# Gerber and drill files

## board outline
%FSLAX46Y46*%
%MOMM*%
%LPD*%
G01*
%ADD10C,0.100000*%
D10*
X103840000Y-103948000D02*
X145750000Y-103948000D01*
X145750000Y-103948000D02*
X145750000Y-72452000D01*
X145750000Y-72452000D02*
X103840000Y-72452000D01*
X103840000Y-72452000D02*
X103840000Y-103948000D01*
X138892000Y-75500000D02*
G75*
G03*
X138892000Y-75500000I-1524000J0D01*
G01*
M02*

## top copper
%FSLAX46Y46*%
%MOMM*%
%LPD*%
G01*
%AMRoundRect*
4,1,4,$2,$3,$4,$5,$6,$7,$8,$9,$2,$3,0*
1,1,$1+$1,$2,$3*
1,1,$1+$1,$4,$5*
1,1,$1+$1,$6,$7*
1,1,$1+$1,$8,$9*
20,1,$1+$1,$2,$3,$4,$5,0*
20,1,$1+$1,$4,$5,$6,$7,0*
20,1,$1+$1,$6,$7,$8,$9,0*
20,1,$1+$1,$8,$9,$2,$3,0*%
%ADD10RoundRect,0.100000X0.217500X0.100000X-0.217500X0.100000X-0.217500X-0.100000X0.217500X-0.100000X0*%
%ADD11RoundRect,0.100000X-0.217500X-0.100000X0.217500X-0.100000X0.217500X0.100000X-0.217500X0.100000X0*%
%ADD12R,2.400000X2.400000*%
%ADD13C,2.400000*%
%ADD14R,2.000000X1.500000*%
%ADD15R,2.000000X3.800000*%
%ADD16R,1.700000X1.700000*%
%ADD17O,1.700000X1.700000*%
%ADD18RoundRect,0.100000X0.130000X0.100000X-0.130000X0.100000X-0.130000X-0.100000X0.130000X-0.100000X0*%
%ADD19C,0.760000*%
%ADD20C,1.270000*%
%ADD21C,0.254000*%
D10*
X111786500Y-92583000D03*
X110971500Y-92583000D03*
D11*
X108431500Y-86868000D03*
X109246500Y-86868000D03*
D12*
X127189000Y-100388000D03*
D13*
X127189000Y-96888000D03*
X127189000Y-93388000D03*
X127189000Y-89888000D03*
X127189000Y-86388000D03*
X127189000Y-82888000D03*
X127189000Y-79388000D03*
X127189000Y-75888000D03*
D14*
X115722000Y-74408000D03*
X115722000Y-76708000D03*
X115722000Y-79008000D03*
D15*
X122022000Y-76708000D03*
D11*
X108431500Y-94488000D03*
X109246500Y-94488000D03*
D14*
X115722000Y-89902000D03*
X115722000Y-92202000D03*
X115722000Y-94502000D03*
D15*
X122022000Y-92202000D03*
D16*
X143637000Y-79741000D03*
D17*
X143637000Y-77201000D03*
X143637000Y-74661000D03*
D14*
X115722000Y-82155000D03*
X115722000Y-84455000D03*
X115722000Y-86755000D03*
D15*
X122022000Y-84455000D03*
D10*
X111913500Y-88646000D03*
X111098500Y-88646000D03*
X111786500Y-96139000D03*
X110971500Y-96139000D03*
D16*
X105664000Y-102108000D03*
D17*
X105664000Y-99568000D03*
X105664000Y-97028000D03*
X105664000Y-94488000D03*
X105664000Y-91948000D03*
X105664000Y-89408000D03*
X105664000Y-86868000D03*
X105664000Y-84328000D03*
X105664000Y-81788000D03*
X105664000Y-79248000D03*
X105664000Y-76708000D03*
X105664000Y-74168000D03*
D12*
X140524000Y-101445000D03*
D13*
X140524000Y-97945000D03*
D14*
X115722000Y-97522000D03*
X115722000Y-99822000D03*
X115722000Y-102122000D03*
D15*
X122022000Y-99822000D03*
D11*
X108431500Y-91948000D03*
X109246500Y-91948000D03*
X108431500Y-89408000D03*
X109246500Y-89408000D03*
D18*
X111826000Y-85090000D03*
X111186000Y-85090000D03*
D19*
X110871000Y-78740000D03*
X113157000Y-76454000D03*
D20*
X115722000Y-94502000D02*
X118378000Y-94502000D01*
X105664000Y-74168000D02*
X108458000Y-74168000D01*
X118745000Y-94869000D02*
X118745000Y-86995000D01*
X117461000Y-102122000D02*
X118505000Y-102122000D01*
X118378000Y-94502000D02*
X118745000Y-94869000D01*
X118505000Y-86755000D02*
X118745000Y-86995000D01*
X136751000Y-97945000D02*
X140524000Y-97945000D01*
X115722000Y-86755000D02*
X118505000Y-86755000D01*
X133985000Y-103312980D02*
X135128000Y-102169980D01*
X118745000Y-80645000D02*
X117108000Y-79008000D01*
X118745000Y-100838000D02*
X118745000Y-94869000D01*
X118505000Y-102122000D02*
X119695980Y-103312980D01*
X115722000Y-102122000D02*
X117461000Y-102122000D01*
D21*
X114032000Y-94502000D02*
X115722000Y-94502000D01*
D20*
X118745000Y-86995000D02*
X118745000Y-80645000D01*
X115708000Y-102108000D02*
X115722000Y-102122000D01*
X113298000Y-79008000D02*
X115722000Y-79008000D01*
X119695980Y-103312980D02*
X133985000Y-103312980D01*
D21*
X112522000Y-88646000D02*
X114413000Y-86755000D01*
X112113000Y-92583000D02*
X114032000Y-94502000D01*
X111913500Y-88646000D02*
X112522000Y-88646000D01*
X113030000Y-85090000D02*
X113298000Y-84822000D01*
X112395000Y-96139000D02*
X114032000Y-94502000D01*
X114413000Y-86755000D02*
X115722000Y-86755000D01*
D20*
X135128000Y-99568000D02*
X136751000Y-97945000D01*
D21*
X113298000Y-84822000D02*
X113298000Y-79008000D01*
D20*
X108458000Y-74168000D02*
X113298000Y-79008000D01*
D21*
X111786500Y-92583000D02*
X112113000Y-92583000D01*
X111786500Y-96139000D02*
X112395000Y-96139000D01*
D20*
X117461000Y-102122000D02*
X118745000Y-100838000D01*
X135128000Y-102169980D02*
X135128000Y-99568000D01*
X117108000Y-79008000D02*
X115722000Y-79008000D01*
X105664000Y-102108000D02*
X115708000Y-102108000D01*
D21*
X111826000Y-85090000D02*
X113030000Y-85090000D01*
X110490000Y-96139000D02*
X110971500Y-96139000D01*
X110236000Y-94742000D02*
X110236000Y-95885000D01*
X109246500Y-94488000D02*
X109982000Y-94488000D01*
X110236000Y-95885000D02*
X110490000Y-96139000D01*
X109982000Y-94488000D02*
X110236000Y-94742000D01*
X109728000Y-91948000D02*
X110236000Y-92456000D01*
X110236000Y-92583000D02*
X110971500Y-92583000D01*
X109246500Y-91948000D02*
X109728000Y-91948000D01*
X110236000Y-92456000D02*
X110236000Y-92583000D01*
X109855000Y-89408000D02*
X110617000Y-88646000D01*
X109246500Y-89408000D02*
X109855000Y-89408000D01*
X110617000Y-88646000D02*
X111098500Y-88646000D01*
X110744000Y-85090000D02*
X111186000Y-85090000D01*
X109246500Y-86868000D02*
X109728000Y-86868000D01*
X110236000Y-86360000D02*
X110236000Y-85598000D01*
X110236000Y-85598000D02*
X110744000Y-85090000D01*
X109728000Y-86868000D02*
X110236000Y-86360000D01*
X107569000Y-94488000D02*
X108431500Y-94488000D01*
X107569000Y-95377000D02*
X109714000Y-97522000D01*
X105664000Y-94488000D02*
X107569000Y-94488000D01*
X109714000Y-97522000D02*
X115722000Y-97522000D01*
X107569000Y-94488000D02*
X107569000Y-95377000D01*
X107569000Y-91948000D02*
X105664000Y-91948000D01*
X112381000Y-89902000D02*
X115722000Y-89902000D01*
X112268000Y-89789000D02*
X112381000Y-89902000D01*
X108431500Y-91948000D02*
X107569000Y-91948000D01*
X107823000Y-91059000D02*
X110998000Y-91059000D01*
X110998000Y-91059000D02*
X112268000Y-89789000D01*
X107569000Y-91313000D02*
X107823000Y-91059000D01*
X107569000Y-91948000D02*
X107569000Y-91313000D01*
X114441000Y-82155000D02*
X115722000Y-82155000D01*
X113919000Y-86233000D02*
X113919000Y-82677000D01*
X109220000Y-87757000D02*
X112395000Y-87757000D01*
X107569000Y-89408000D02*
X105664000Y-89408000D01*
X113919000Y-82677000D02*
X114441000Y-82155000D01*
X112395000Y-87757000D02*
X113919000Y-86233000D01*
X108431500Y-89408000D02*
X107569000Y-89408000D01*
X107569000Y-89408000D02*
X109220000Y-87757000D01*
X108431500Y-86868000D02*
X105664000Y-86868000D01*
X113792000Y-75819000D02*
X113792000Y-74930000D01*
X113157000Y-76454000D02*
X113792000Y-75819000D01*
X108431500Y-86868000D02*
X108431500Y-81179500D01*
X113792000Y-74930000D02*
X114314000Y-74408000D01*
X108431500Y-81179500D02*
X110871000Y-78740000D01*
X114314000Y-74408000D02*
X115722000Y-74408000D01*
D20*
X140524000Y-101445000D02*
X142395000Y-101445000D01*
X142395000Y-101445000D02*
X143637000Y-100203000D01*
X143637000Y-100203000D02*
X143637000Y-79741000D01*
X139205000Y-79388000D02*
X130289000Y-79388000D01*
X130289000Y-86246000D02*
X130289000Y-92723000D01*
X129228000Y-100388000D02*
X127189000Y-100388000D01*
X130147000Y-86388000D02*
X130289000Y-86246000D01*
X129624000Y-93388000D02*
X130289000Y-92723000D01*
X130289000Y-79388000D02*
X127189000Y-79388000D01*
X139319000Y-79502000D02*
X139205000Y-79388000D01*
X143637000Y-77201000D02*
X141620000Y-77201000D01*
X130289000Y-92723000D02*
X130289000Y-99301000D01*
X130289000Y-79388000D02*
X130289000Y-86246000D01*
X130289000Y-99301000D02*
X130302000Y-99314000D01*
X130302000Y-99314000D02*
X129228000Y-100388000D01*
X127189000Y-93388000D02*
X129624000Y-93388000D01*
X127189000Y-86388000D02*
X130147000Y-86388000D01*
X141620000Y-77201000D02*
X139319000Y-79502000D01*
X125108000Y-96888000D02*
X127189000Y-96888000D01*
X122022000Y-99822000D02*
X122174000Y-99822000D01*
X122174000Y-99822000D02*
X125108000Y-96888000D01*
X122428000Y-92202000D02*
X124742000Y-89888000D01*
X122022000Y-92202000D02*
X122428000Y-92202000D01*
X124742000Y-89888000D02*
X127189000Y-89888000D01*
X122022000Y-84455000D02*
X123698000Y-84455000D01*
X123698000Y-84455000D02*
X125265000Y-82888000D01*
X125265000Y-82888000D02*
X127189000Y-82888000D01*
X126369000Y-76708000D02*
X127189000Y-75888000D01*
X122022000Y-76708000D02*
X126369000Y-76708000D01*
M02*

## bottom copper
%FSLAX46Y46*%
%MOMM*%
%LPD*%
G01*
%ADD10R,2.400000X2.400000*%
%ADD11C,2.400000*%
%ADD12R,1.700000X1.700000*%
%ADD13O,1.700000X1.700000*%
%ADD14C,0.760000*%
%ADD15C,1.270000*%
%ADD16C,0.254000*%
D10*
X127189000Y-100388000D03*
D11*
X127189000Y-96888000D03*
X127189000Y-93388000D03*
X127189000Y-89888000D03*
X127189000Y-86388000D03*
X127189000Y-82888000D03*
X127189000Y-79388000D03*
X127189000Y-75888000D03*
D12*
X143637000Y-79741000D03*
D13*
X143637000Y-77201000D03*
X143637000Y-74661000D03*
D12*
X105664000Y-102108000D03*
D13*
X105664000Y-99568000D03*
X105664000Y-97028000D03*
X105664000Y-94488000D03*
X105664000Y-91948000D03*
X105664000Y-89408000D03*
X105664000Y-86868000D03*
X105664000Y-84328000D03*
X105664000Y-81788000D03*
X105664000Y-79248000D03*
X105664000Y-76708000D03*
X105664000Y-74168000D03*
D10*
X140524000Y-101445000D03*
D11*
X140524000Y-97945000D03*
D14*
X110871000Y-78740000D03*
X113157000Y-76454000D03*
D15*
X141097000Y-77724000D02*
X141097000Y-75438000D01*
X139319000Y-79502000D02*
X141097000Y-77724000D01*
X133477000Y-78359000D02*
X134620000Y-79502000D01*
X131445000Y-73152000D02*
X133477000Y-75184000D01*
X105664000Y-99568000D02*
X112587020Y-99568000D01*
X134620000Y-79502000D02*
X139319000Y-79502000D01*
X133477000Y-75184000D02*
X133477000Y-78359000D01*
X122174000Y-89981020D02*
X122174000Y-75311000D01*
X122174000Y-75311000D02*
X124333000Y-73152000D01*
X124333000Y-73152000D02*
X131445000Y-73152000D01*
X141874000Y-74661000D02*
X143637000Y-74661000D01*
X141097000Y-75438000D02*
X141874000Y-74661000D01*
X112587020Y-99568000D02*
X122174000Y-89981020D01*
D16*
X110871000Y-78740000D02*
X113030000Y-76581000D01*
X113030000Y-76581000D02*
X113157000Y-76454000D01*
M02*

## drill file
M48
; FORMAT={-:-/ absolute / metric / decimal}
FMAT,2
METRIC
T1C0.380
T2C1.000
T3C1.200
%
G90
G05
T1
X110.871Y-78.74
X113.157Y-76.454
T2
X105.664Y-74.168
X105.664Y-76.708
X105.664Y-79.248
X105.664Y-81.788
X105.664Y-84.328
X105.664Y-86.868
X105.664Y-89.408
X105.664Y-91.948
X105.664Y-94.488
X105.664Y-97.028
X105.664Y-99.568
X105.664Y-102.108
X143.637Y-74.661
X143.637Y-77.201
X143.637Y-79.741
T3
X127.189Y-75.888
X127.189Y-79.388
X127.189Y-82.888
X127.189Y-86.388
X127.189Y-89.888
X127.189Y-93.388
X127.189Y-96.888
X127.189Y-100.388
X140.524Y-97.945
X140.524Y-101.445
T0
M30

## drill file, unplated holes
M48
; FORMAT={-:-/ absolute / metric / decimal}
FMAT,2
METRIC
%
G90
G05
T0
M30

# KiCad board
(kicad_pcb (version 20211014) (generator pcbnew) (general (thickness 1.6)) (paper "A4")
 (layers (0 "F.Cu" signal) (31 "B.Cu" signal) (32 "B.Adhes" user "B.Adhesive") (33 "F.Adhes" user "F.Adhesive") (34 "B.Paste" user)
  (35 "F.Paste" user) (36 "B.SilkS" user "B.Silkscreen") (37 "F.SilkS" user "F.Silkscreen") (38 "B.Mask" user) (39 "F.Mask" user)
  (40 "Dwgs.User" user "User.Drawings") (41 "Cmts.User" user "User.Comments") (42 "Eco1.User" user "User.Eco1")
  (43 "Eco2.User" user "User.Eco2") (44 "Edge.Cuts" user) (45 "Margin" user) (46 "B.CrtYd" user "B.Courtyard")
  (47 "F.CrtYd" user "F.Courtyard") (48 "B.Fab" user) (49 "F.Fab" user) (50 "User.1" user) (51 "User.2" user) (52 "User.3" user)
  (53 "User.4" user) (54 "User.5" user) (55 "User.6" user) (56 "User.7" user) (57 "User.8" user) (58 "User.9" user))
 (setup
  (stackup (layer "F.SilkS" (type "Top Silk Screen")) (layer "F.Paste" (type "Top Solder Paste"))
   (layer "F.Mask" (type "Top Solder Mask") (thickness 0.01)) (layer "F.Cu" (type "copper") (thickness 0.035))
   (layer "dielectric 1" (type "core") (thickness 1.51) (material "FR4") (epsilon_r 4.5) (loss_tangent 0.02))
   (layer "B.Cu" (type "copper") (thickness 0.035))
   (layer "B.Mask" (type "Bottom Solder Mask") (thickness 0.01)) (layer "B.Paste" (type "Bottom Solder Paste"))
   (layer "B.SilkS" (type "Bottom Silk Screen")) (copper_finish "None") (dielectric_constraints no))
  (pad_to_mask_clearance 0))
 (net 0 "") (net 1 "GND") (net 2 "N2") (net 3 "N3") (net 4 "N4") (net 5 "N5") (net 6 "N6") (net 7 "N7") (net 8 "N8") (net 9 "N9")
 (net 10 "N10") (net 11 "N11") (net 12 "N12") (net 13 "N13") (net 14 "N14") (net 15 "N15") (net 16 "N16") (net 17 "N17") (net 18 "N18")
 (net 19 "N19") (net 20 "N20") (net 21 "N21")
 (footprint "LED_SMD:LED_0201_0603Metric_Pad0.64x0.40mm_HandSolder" (layer "F.Cu") (at 111.379 92.583 180)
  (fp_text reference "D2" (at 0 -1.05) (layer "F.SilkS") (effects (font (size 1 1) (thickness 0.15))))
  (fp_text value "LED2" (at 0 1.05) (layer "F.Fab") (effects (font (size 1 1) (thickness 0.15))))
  (pad "" smd roundrect locked (at 0.4325 0 180) (size 0.458 0.36) (layers "F.Paste") (roundrect_rratio 0.25))
  (pad "" smd roundrect locked (at -0.4325 0 180) (size 0.458 0.36) (layers "F.Paste") (roundrect_rratio 0.25))
  (pad "1" smd roundrect locked (at -0.4075 0 180) (size 0.635 0.4) (layers "F.Cu" "F.Mask") (roundrect_rratio 0.25) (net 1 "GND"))
  (pad "2" smd roundrect locked (at 0.4075 0 180) (size 0.635 0.4) (layers "F.Cu" "F.Mask") (roundrect_rratio 0.25) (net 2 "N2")))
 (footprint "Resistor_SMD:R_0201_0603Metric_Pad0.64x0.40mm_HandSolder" (layer "F.Cu") (at 108.839 86.868)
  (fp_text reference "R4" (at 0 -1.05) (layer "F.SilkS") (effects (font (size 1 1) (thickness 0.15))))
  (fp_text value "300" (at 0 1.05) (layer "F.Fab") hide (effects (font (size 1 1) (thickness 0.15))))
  (pad "" smd roundrect locked (at 0.4325 0) (size 0.458 0.36) (layers "F.Paste") (roundrect_rratio 0.25))
  (pad "" smd roundrect locked (at -0.4325 0) (size 0.458 0.36) (layers "F.Paste") (roundrect_rratio 0.25))
  (pad "1" smd roundrect locked (at -0.4075 0) (size 0.635 0.4) (layers "F.Cu" "F.Mask") (roundrect_rratio 0.25) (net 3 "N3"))
  (pad "2" smd roundrect locked (at 0.4075 0) (size 0.635 0.4) (layers "F.Cu" "F.Mask") (roundrect_rratio 0.25) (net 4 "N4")))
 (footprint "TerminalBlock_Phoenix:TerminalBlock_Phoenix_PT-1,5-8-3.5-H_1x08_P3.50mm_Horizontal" (layer "F.Cu") (at 127.189 100.388 90)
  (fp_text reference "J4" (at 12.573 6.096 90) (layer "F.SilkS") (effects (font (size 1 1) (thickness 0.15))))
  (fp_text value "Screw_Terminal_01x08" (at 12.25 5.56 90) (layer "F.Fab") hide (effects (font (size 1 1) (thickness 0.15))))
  (pad "1" thru_hole rect locked (at 0 0 90) (size 2.4 2.4) (drill 1.2) (layers *.Cu *.Mask) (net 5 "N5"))
  (pad "2" thru_hole circle locked (at 3.5 0 90) (size 2.4 2.4) (drill 1.2) (layers *.Cu *.Mask) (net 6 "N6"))
  (pad "3" thru_hole circle locked (at 7 0 90) (size 2.4 2.4) (drill 1.2) (layers *.Cu *.Mask) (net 5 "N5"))
  (pad "4" thru_hole circle locked (at 10.5 0 90) (size 2.4 2.4) (drill 1.2) (layers *.Cu *.Mask) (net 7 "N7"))
  (pad "5" thru_hole circle locked (at 14 0 90) (size 2.4 2.4) (drill 1.2) (layers *.Cu *.Mask) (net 5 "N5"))
  (pad "6" thru_hole circle locked (at 17.5 0 90) (size 2.4 2.4) (drill 1.2) (layers *.Cu *.Mask) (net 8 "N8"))
  (pad "7" thru_hole circle locked (at 21 0 90) (size 2.4 2.4) (drill 1.2) (layers *.Cu *.Mask) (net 5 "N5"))
  (pad "8" thru_hole circle locked (at 24.5 0 90) (size 2.4 2.4) (drill 1.2) (layers *.Cu *.Mask) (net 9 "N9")))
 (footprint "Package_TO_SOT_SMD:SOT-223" (layer "F.Cu") (at 118.872 76.708)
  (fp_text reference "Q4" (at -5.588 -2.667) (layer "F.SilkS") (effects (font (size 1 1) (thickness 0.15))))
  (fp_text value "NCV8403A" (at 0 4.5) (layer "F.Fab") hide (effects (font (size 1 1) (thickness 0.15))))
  (pad "1" smd rect locked (at -3.15 -2.3) (size 2 1.5) (layers "F.Cu" "F.Paste" "F.Mask") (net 3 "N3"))
  (pad "2" smd rect locked (at -3.15 0) (size 2 1.5) (layers "F.Cu" "F.Paste" "F.Mask"))
  (pad "3" smd rect locked (at -3.15 2.3) (size 2 1.5) (layers "F.Cu" "F.Paste" "F.Mask") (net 1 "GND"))
  (pad "4" smd rect locked (at 3.15 0) (size 2 3.8) (layers "F.Cu" "F.Paste" "F.Mask") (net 9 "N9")))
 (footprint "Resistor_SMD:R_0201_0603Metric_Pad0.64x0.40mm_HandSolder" (layer "F.Cu") (at 108.839 94.488)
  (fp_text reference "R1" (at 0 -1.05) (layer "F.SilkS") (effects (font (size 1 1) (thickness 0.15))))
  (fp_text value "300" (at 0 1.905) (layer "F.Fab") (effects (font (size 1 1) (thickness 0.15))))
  (pad "" smd roundrect locked (at -0.4325 0) (size 0.458 0.36) (layers "F.Paste") (roundrect_rratio 0.25))
  (pad "" smd roundrect locked (at 0.4325 0) (size 0.458 0.36) (layers "F.Paste") (roundrect_rratio 0.25))
  (pad "1" smd roundrect locked (at -0.4075 0) (size 0.635 0.4) (layers "F.Cu" "F.Mask") (roundrect_rratio 0.25) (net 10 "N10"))
  (pad "2" smd roundrect locked (at 0.4075 0) (size 0.635 0.4) (layers "F.Cu" "F.Mask") (roundrect_rratio 0.25) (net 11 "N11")))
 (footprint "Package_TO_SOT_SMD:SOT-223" (layer "F.Cu") (at 118.872 92.202)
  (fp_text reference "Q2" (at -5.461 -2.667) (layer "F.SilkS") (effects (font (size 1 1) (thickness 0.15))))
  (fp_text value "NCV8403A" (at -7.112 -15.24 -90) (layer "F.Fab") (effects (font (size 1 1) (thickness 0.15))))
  (pad "1" smd rect locked (at -3.15 -2.3) (size 2 1.5) (layers "F.Cu" "F.Paste" "F.Mask") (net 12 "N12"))
  (pad "2" smd rect locked (at -3.15 0) (size 2 1.5) (layers "F.Cu" "F.Paste" "F.Mask"))
  (pad "3" smd rect locked (at -3.15 2.3) (size 2 1.5) (layers "F.Cu" "F.Paste" "F.Mask") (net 1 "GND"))
  (pad "4" smd rect locked (at 3.15 0) (size 2 3.8) (layers "F.Cu" "F.Paste" "F.Mask") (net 7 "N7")))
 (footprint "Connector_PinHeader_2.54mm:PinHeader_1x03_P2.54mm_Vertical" (layer "F.Cu") (at 143.637 79.741 180)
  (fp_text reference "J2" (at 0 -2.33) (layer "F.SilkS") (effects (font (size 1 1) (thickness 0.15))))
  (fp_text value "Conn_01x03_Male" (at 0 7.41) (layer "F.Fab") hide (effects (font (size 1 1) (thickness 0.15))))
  (pad "1" thru_hole rect locked (at 0 0 180) (size 1.7 1.7) (drill 1) (layers *.Cu *.Mask) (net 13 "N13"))
  (pad "2" thru_hole oval locked (at 0 2.54 180) (size 1.7 1.7) (drill 1) (layers *.Cu *.Mask) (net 5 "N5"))
  (pad "3" thru_hole oval locked (at 0 5.08 180) (size 1.7 1.7) (drill 1) (layers *.Cu *.Mask) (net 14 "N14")))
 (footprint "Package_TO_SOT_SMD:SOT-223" (layer "F.Cu") (at 118.872 84.455)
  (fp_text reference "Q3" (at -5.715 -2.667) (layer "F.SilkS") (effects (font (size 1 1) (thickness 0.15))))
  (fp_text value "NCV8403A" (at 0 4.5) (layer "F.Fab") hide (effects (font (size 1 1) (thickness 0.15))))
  (pad "1" smd rect locked (at -3.15 -2.3) (size 2 1.5) (layers "F.Cu" "F.Paste" "F.Mask") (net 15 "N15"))
  (pad "2" smd rect locked (at -3.15 0) (size 2 1.5) (layers "F.Cu" "F.Paste" "F.Mask"))
  (pad "3" smd rect locked (at -3.15 2.3) (size 2 1.5) (layers "F.Cu" "F.Paste" "F.Mask") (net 1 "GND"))
  (pad "4" smd rect locked (at 3.15 0) (size 2 3.8) (layers "F.Cu" "F.Paste" "F.Mask") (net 8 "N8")))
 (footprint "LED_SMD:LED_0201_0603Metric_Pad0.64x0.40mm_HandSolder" (layer "F.Cu") (at 111.506 88.646 180)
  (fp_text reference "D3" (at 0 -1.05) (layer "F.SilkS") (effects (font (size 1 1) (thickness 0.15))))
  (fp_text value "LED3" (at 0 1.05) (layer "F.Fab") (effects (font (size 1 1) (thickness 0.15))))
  (pad "" smd roundrect locked (at 0.4325 0 180) (size 0.458 0.36) (layers "F.Paste") (roundrect_rratio 0.25))
  (pad "" smd roundrect locked (at -0.4325 0 180) (size 0.458 0.36) (layers "F.Paste") (roundrect_rratio 0.25))
  (pad "1" smd roundrect locked (at -0.4075 0 180) (size 0.635 0.4) (layers "F.Cu" "F.Mask") (roundrect_rratio 0.25) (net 1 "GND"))
  (pad "2" smd roundrect locked (at 0.4075 0 180) (size 0.635 0.4) (layers "F.Cu" "F.Mask") (roundrect_rratio 0.25) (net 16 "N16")))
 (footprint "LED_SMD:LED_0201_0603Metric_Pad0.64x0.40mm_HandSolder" (layer "F.Cu") (at 111.379 96.139 180)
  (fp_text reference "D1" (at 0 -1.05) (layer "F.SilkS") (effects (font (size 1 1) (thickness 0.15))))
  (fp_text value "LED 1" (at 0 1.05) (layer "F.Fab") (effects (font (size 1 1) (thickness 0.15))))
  (pad "" smd roundrect locked (at 0.4325 0 180) (size 0.458 0.36) (layers "F.Paste") (roundrect_rratio 0.25))
  (pad "" smd roundrect locked (at -0.4325 0 180) (size 0.458 0.36) (layers "F.Paste") (roundrect_rratio 0.25))
  (pad "1" smd roundrect locked (at -0.4075 0 180) (size 0.635 0.4) (layers "F.Cu" "F.Mask") (roundrect_rratio 0.25) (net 1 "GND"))
  (pad "2" smd roundrect locked (at 0.4075 0 180) (size 0.635 0.4) (layers "F.Cu" "F.Mask") (roundrect_rratio 0.25) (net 11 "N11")))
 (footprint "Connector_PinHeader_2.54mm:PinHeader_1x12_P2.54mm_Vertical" (layer "F.Cu") (at 105.664 102.108 180)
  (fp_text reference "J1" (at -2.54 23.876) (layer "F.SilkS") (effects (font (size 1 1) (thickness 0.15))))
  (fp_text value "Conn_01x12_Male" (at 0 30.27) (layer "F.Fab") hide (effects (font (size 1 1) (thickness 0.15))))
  (pad "1" thru_hole rect locked (at 0 0 180) (size 1.7 1.7) (drill 1) (layers *.Cu *.Mask) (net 1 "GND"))
  (pad "2" thru_hole oval locked (at 0 2.54 180) (size 1.7 1.7) (drill 1) (layers *.Cu *.Mask) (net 14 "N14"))
  (pad "3" thru_hole oval locked (at 0 5.08 180) (size 1.7 1.7) (drill 1) (layers *.Cu *.Mask) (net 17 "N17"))
  (pad "4" thru_hole oval locked (at 0 7.62 180) (size 1.7 1.7) (drill 1) (layers *.Cu *.Mask) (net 10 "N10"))
  (pad "5" thru_hole oval locked (at 0 10.16 180) (size 1.7 1.7) (drill 1) (layers *.Cu *.Mask) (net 12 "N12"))
  (pad "6" thru_hole oval locked (at 0 12.7 180) (size 1.7 1.7) (drill 1) (layers *.Cu *.Mask) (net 15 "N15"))
  (pad "7" thru_hole oval locked (at 0 15.24 180) (size 1.7 1.7) (drill 1) (layers *.Cu *.Mask) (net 3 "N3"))
  (pad "8" thru_hole oval locked (at 0 17.78 180) (size 1.7 1.7) (drill 1) (layers *.Cu *.Mask) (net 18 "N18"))
  (pad "9" thru_hole oval locked (at 0 20.32 180) (size 1.7 1.7) (drill 1) (layers *.Cu *.Mask) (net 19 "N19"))
  (pad "10" thru_hole oval locked (at 0 22.86 180) (size 1.7 1.7) (drill 1) (layers *.Cu *.Mask) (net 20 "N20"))
  (pad "11" thru_hole oval locked (at 0 25.4 180) (size 1.7 1.7) (drill 1) (layers *.Cu *.Mask) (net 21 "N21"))
  (pad "12" thru_hole oval locked (at 0 27.94 180) (size 1.7 1.7) (drill 1) (layers *.Cu *.Mask) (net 1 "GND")))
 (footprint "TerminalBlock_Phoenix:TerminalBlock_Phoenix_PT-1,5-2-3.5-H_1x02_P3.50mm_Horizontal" (layer "F.Cu") (at 140.524 101.445 90)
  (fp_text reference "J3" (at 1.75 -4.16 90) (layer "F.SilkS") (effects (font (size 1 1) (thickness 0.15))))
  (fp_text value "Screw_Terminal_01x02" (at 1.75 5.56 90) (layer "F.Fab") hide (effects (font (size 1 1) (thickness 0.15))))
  (pad "1" thru_hole rect locked (at 0 0 90) (size 2.4 2.4) (drill 1.2) (layers *.Cu *.Mask) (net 13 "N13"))
  (pad "2" thru_hole circle locked (at 3.5 0 90) (size 2.4 2.4) (drill 1.2) (layers *.Cu *.Mask) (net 1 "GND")))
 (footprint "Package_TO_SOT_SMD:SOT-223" (layer "F.Cu") (at 118.872 99.822)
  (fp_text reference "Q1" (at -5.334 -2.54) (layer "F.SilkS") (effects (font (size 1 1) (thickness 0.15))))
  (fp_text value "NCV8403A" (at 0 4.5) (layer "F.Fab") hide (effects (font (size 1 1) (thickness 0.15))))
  (pad "1" smd rect locked (at -3.15 -2.3) (size 2 1.5) (layers "F.Cu" "F.Paste" "F.Mask") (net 10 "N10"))
  (pad "2" smd rect locked (at -3.15 0) (size 2 1.5) (layers "F.Cu" "F.Paste" "F.Mask"))
  (pad "3" smd rect locked (at -3.15 2.3) (size 2 1.5) (layers "F.Cu" "F.Paste" "F.Mask") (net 1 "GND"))
  (pad "4" smd rect locked (at 3.15 0) (size 2 3.8) (layers "F.Cu" "F.Paste" "F.Mask") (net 6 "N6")))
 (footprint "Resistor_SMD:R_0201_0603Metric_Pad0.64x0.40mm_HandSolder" (layer "F.Cu") (at 108.839 91.948)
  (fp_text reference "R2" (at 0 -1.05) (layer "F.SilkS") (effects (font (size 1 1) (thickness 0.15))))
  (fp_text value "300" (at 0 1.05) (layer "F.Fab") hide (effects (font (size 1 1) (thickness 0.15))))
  (pad "" smd roundrect locked (at 0.4325 0) (size 0.458 0.36) (layers "F.Paste") (roundrect_rratio 0.25))
  (pad "" smd roundrect locked (at -0.4325 0) (size 0.458 0.36) (layers "F.Paste") (roundrect_rratio 0.25))
  (pad "1" smd roundrect locked (at -0.4075 0) (size 0.635 0.4) (layers "F.Cu" "F.Mask") (roundrect_rratio 0.25) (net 12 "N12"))
  (pad "2" smd roundrect locked (at 0.4075 0) (size 0.635 0.4) (layers "F.Cu" "F.Mask") (roundrect_rratio 0.25) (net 2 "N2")))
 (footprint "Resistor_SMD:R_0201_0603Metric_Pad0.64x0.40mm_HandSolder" (layer "F.Cu") (at 108.839 89.408)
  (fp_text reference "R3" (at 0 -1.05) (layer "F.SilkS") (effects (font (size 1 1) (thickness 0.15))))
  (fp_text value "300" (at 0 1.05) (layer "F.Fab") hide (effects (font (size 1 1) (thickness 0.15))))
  (pad "" smd roundrect locked (at 0.4325 0) (size 0.458 0.36) (layers "F.Paste") (roundrect_rratio 0.25))
  (pad "" smd roundrect locked (at -0.4325 0) (size 0.458 0.36) (layers "F.Paste") (roundrect_rratio 0.25))
  (pad "1" smd roundrect locked (at -0.4075 0) (size 0.635 0.4) (layers "F.Cu" "F.Mask") (roundrect_rratio 0.25) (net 15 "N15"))
  (pad "2" smd roundrect locked (at 0.4075 0) (size 0.635 0.4) (layers "F.Cu" "F.Mask") (roundrect_rratio 0.25) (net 16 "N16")))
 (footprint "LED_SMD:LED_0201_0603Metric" (layer "F.Cu") (at 111.506 85.09 180)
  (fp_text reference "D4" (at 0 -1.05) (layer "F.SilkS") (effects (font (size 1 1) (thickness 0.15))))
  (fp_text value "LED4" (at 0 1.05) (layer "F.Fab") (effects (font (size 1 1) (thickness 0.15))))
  (pad "" smd roundrect locked (at 0.345 0 180) (size 0.318 0.36) (layers "F.Paste") (roundrect_rratio 0.25))
  (pad "" smd roundrect locked (at -0.345 0 180) (size 0.318 0.36) (layers "F.Paste") (roundrect_rratio 0.25))
  (pad "1" smd roundrect locked (at -0.32 0 180) (size 0.46 0.4) (layers "F.Cu" "F.Mask") (roundrect_rratio 0.25) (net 1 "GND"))
  (pad "2" smd roundrect locked (at 0.32 0 180) (size 0.46 0.4) (layers "F.Cu" "F.Mask") (roundrect_rratio 0.25) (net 4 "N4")))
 (gr_rect (start 103.84 103.948) (end 145.75 72.452) (layer "Edge.Cuts") (width 0.1) (fill none))
 (gr_circle (center 137.368 75.5) (end 135.844 75.5) (layer "Edge.Cuts") (width 0.1) (fill none))
 (segment (start 115.722 94.502) (end 118.378 94.502) (width 1.27) (layer "F.Cu") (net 1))
 (segment (start 105.664 74.168) (end 108.458 74.168) (width 1.27) (layer "F.Cu") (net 1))
 (segment (start 118.745 94.869) (end 118.745 86.995) (width 1.27) (layer "F.Cu") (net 1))
 (segment (start 117.461 102.122) (end 118.505 102.122) (width 1.27) (layer "F.Cu") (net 1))
 (segment (start 118.378 94.502) (end 118.745 94.869) (width 1.27) (layer "F.Cu") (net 1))
 (segment (start 118.505 86.755) (end 118.745 86.995) (width 1.27) (layer "F.Cu") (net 1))
 (segment (start 136.751 97.945) (end 140.524 97.945) (width 1.27) (layer "F.Cu") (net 1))
 (segment (start 115.722 86.755) (end 118.505 86.755) (width 1.27) (layer "F.Cu") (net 1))
 (segment (start 133.985 103.31298) (end 135.128 102.16998) (width 1.27) (layer "F.Cu") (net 1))
 (segment (start 118.745 80.645) (end 117.108 79.008) (width 1.27) (layer "F.Cu") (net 1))
 (segment (start 118.745 100.838) (end 118.745 94.869) (width 1.27) (layer "F.Cu") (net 1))
 (segment (start 118.505 102.122) (end 119.69598 103.31298) (width 1.27) (layer "F.Cu") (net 1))
 (segment (start 115.722 102.122) (end 117.461 102.122) (width 1.27) (layer "F.Cu") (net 1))
 (segment (start 114.032 94.502) (end 115.722 94.502) (width 0.254) (layer "F.Cu") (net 1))
 (segment (start 118.745 86.995) (end 118.745 80.645) (width 1.27) (layer "F.Cu") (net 1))
 (segment (start 115.708 102.108) (end 115.722 102.122) (width 1.27) (layer "F.Cu") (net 1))
 (segment (start 113.298 79.008) (end 115.722 79.008) (width 1.27) (layer "F.Cu") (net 1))
 (segment (start 119.69598 103.31298) (end 133.985 103.31298) (width 1.27) (layer "F.Cu") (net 1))
 (segment (start 112.522 88.646) (end 114.413 86.755) (width 0.254) (layer "F.Cu") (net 1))
 (segment (start 112.113 92.583) (end 114.032 94.502) (width 0.254) (layer "F.Cu") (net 1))
 (segment (start 111.9135 88.646) (end 112.522 88.646) (width 0.254) (layer "F.Cu") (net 1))
 (segment (start 113.03 85.09) (end 113.298 84.822) (width 0.254) (layer "F.Cu") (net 1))
 (segment (start 112.395 96.139) (end 114.032 94.502) (width 0.254) (layer "F.Cu") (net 1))
 (segment (start 114.413 86.755) (end 115.722 86.755) (width 0.254) (layer "F.Cu") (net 1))
 (segment (start 135.128 99.568) (end 136.751 97.945) (width 1.27) (layer "F.Cu") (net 1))
 (segment (start 113.298 84.822) (end 113.298 79.008) (width 0.254) (layer "F.Cu") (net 1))
 (segment (start 108.458 74.168) (end 113.298 79.008) (width 1.27) (layer "F.Cu") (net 1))
 (segment (start 111.7865 92.583) (end 112.113 92.583) (width 0.254) (layer "F.Cu") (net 1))
 (segment (start 111.7865 96.139) (end 112.395 96.139) (width 0.254) (layer "F.Cu") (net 1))
 (segment (start 117.461 102.122) (end 118.745 100.838) (width 1.27) (layer "F.Cu") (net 1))
 (segment (start 135.128 102.16998) (end 135.128 99.568) (width 1.27) (layer "F.Cu") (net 1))
 (segment (start 117.108 79.008) (end 115.722 79.008) (width 1.27) (layer "F.Cu") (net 1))
 (segment (start 105.664 102.108) (end 115.708 102.108) (width 1.27) (layer "F.Cu") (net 1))
 (segment (start 111.826 85.09) (end 113.03 85.09) (width 0.254) (layer "F.Cu") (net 1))
 (segment (start 110.49 96.139) (end 110.9715 96.139) (width 0.254) (layer "F.Cu") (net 11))
 (segment (start 110.236 94.742) (end 110.236 95.885) (width 0.254) (layer "F.Cu") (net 11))
 (segment (start 109.2465 94.488) (end 109.982 94.488) (width 0.254) (layer "F.Cu") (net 11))
 (segment (start 110.236 95.885) (end 110.49 96.139) (width 0.254) (layer "F.Cu") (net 11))
 (segment (start 109.982 94.488) (end 110.236 94.742) (width 0.254) (layer "F.Cu") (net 11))
 (segment (start 109.728 91.948) (end 110.236 92.456) (width 0.254) (layer "F.Cu") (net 2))
 (segment (start 110.236 92.583) (end 110.9715 92.583) (width 0.254) (layer "F.Cu") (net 2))
 (segment (start 109.2465 91.948) (end 109.728 91.948) (width 0.254) (layer "F.Cu") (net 2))
 (segment (start 110.236 92.456) (end 110.236 92.583) (width 0.254) (layer "F.Cu") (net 2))
 (segment (start 109.855 89.408) (end 110.617 88.646) (width 0.254) (layer "F.Cu") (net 16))
 (segment (start 109.2465 89.408) (end 109.855 89.408) (width 0.254) (layer "F.Cu") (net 16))
 (segment (start 110.617 88.646) (end 111.0985 88.646) (width 0.254) (layer "F.Cu") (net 16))
 (segment (start 110.744 85.09) (end 111.186 85.09) (width 0.254) (layer "F.Cu") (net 4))
 (segment (start 109.2465 86.868) (end 109.728 86.868) (width 0.254) (layer "F.Cu") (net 4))
 (segment (start 110.236 86.36) (end 110.236 85.598) (width 0.254) (layer "F.Cu") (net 4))
 (segment (start 110.236 85.598) (end 110.744 85.09) (width 0.254) (layer "F.Cu") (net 4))
 (segment (start 109.728 86.868) (end 110.236 86.36) (width 0.254) (layer "F.Cu") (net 4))
 (segment (start 141.097 77.724) (end 141.097 75.438) (width 1.27) (layer "B.Cu") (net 14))
 (segment (start 139.319 79.502) (end 141.097 77.724) (width 1.27) (layer "B.Cu") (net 14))
 (segment (start 133.477 78.359) (end 134.62 79.502) (width 1.27) (layer "B.Cu") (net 14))
 (segment (start 131.445 73.152) (end 133.477 75.184) (width 1.27) (layer "B.Cu") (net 14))
 (segment (start 105.664 99.568) (end 112.58702 99.568) (width 1.27) (layer "B.Cu") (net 14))
 (segment (start 134.62 79.502) (end 139.319 79.502) (width 1.27) (layer "B.Cu") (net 14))
 (segment (start 133.477 75.184) (end 133.477 78.359) (width 1.27) (layer "B.Cu") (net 14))
 (segment (start 122.174 89.98102) (end 122.174 75.311) (width 1.27) (layer "B.Cu") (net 14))
 (segment (start 122.174 75.311) (end 124.333 73.152) (width 1.27) (layer "B.Cu") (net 14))
 (segment (start 124.333 73.152) (end 131.445 73.152) (width 1.27) (layer "B.Cu") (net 14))
 (segment (start 141.874 74.661) (end 143.637 74.661) (width 1.27) (layer "B.Cu") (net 14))
 (segment (start 141.097 75.438) (end 141.874 74.661) (width 1.27) (layer "B.Cu") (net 14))
 (segment (start 112.58702 99.568) (end 122.174 89.98102) (width 1.27) (layer "B.Cu") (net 14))
 (segment (start 107.569 94.488) (end 108.4315 94.488) (width 0.254) (layer "F.Cu") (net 10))
 (segment (start 107.569 95.377) (end 109.714 97.522) (width 0.254) (layer "F.Cu") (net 10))
 (segment (start 105.664 94.488) (end 107.569 94.488) (width 0.254) (layer "F.Cu") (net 10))
 (segment (start 109.714 97.522) (end 115.722 97.522) (width 0.254) (layer "F.Cu") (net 10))
 (segment (start 107.569 94.488) (end 107.569 95.377) (width 0.254) (layer "F.Cu") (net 10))
 (segment (start 107.569 91.948) (end 105.664 91.948) (width 0.254) (layer "F.Cu") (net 12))
 (segment (start 112.381 89.902) (end 115.722 89.902) (width 0.254) (layer "F.Cu") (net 12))
 (segment (start 112.268 89.789) (end 112.381 89.902) (width 0.254) (layer "F.Cu") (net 12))
 (segment (start 108.4315 91.948) (end 107.569 91.948) (width 0.254) (layer "F.Cu") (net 12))
 (segment (start 107.823 91.059) (end 110.998 91.059) (width 0.254) (layer "F.Cu") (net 12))
 (segment (start 110.998 91.059) (end 112.268 89.789) (width 0.254) (layer "F.Cu") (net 12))
 (segment (start 107.569 91.313) (end 107.823 91.059) (width 0.254) (layer "F.Cu") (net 12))
 (segment (start 107.569 91.948) (end 107.569 91.313) (width 0.254) (layer "F.Cu") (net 12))
 (segment (start 114.441 82.155) (end 115.722 82.155) (width 0.254) (layer "F.Cu") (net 15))
 (segment (start 113.919 86.233) (end 113.919 82.677) (width 0.254) (layer "F.Cu") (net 15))
 (segment (start 109.22 87.757) (end 112.395 87.757) (width 0.254) (layer "F.Cu") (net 15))
 (segment (start 107.569 89.408) (end 105.664 89.408) (width 0.254) (layer "F.Cu") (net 15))
 (segment (start 113.919 82.677) (end 114.441 82.155) (width 0.254) (layer "F.Cu") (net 15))
 (segment (start 112.395 87.757) (end 113.919 86.233) (width 0.254) (layer "F.Cu") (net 15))
 (segment (start 108.4315 89.408) (end 107.569 89.408) (width 0.254) (layer "F.Cu") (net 15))
 (segment (start 107.569 89.408) (end 109.22 87.757) (width 0.254) (layer "F.Cu") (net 15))
 (segment (start 108.4315 86.868) (end 105.664 86.868) (width 0.254) (layer "F.Cu") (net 3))
 (segment (start 113.792 75.819) (end 113.792 74.93) (width 0.254) (layer "F.Cu") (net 3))
 (segment (start 113.157 76.454) (end 113.792 75.819) (width 0.254) (layer "F.Cu") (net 3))
 (segment (start 108.4315 86.868) (end 108.4315 81.1795) (width 0.254) (layer "F.Cu") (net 3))
 (segment (start 113.792 74.93) (end 114.314 74.408) (width 0.254) (layer "F.Cu") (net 3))
 (segment (start 108.4315 81.1795) (end 110.871 78.74) (width 0.254) (layer "F.Cu") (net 3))
 (segment (start 114.314 74.408) (end 115.722 74.408) (width 0.254) (layer "F.Cu") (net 3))
 (via (at 110.871 78.74) (size 0.76) (drill 0.38) (layers "F.Cu" "B.Cu") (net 3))
 (via (at 113.157 76.454) (size 0.76) (drill 0.38) (layers "F.Cu" "B.Cu") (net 3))
 (segment (start 110.871 78.74) (end 113.03 76.581) (width 0.254) (layer "B.Cu") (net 3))
 (segment (start 113.03 76.581) (end 113.157 76.454) (width 0.254) (layer "B.Cu") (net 3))
 (segment (start 140.524 101.445) (end 142.395 101.445) (width 1.27) (layer "F.Cu") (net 13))
 (segment (start 142.395 101.445) (end 143.637 100.203) (width 1.27) (layer "F.Cu") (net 13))
 (segment (start 143.637 100.203) (end 143.637 79.741) (width 1.27) (layer "F.Cu") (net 13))
 (segment (start 139.205 79.388) (end 130.289 79.388) (width 1.27) (layer "F.Cu") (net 5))
 (segment (start 130.289 86.246) (end 130.289 92.723) (width 1.27) (layer "F.Cu") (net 5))
 (segment (start 129.228 100.388) (end 127.189 100.388) (width 1.27) (layer "F.Cu") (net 5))
 (segment (start 130.147 86.388) (end 130.289 86.246) (width 1.27) (layer "F.Cu") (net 5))
 (segment (start 129.624 93.388) (end 130.289 92.723) (width 1.27) (layer "F.Cu") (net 5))
 (segment (start 130.289 79.388) (end 127.189 79.388) (width 1.27) (layer "F.Cu") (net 5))
 (segment (start 139.319 79.502) (end 139.205 79.388) (width 1.27) (layer "F.Cu") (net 5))
 (segment (start 143.637 77.201) (end 141.62 77.201) (width 1.27) (layer "F.Cu") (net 5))
 (segment (start 130.289 92.723) (end 130.289 99.301) (width 1.27) (layer "F.Cu") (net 5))
 (segment (start 130.289 79.388) (end 130.289 86.246) (width 1.27) (layer "F.Cu") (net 5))
 (segment (start 130.289 99.301) (end 130.302 99.314) (width 1.27) (layer "F.Cu") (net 5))
 (segment (start 130.302 99.314) (end 129.228 100.388) (width 1.27) (layer "F.Cu") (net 5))
 (segment (start 127.189 93.388) (end 129.624 93.388) (width 1.27) (layer "F.Cu") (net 5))
 (segment (start 127.189 86.388) (end 130.147 86.388) (width 1.27) (layer "F.Cu") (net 5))
 (segment (start 141.62 77.201) (end 139.319 79.502) (width 1.27) (layer "F.Cu") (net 5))
 (segment (start 125.108 96.888) (end 127.189 96.888) (width 1.27) (layer "F.Cu") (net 6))
 (segment (start 122.022 99.822) (end 122.174 99.822) (width 1.27) (layer "F.Cu") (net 6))
 (segment (start 122.174 99.822) (end 125.108 96.888) (width 1.27) (layer "F.Cu") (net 6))
 (segment (start 122.428 92.202) (end 124.742 89.888) (width 1.27) (layer "F.Cu") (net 7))
 (segment (start 122.022 92.202) (end 122.428 92.202) (width 1.27) (layer "F.Cu") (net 7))
 (segment (start 124.742 89.888) (end 127.189 89.888) (width 1.27) (layer "F.Cu") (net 7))
 (segment (start 122.022 84.455) (end 123.698 84.455) (width 1.27) (layer "F.Cu") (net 8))
 (segment (start 123.698 84.455) (end 125.265 82.888) (width 1.27) (layer "F.Cu") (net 8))
 (segment (start 125.265 82.888) (end 127.189 82.888) (width 1.27) (layer "F.Cu") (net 8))
 (segment (start 126.369 76.708) (end 127.189 75.888) (width 1.27) (layer "F.Cu") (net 9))
 (segment (start 122.022 76.708) (end 126.369 76.708) (width 1.27) (layer "F.Cu") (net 9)))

